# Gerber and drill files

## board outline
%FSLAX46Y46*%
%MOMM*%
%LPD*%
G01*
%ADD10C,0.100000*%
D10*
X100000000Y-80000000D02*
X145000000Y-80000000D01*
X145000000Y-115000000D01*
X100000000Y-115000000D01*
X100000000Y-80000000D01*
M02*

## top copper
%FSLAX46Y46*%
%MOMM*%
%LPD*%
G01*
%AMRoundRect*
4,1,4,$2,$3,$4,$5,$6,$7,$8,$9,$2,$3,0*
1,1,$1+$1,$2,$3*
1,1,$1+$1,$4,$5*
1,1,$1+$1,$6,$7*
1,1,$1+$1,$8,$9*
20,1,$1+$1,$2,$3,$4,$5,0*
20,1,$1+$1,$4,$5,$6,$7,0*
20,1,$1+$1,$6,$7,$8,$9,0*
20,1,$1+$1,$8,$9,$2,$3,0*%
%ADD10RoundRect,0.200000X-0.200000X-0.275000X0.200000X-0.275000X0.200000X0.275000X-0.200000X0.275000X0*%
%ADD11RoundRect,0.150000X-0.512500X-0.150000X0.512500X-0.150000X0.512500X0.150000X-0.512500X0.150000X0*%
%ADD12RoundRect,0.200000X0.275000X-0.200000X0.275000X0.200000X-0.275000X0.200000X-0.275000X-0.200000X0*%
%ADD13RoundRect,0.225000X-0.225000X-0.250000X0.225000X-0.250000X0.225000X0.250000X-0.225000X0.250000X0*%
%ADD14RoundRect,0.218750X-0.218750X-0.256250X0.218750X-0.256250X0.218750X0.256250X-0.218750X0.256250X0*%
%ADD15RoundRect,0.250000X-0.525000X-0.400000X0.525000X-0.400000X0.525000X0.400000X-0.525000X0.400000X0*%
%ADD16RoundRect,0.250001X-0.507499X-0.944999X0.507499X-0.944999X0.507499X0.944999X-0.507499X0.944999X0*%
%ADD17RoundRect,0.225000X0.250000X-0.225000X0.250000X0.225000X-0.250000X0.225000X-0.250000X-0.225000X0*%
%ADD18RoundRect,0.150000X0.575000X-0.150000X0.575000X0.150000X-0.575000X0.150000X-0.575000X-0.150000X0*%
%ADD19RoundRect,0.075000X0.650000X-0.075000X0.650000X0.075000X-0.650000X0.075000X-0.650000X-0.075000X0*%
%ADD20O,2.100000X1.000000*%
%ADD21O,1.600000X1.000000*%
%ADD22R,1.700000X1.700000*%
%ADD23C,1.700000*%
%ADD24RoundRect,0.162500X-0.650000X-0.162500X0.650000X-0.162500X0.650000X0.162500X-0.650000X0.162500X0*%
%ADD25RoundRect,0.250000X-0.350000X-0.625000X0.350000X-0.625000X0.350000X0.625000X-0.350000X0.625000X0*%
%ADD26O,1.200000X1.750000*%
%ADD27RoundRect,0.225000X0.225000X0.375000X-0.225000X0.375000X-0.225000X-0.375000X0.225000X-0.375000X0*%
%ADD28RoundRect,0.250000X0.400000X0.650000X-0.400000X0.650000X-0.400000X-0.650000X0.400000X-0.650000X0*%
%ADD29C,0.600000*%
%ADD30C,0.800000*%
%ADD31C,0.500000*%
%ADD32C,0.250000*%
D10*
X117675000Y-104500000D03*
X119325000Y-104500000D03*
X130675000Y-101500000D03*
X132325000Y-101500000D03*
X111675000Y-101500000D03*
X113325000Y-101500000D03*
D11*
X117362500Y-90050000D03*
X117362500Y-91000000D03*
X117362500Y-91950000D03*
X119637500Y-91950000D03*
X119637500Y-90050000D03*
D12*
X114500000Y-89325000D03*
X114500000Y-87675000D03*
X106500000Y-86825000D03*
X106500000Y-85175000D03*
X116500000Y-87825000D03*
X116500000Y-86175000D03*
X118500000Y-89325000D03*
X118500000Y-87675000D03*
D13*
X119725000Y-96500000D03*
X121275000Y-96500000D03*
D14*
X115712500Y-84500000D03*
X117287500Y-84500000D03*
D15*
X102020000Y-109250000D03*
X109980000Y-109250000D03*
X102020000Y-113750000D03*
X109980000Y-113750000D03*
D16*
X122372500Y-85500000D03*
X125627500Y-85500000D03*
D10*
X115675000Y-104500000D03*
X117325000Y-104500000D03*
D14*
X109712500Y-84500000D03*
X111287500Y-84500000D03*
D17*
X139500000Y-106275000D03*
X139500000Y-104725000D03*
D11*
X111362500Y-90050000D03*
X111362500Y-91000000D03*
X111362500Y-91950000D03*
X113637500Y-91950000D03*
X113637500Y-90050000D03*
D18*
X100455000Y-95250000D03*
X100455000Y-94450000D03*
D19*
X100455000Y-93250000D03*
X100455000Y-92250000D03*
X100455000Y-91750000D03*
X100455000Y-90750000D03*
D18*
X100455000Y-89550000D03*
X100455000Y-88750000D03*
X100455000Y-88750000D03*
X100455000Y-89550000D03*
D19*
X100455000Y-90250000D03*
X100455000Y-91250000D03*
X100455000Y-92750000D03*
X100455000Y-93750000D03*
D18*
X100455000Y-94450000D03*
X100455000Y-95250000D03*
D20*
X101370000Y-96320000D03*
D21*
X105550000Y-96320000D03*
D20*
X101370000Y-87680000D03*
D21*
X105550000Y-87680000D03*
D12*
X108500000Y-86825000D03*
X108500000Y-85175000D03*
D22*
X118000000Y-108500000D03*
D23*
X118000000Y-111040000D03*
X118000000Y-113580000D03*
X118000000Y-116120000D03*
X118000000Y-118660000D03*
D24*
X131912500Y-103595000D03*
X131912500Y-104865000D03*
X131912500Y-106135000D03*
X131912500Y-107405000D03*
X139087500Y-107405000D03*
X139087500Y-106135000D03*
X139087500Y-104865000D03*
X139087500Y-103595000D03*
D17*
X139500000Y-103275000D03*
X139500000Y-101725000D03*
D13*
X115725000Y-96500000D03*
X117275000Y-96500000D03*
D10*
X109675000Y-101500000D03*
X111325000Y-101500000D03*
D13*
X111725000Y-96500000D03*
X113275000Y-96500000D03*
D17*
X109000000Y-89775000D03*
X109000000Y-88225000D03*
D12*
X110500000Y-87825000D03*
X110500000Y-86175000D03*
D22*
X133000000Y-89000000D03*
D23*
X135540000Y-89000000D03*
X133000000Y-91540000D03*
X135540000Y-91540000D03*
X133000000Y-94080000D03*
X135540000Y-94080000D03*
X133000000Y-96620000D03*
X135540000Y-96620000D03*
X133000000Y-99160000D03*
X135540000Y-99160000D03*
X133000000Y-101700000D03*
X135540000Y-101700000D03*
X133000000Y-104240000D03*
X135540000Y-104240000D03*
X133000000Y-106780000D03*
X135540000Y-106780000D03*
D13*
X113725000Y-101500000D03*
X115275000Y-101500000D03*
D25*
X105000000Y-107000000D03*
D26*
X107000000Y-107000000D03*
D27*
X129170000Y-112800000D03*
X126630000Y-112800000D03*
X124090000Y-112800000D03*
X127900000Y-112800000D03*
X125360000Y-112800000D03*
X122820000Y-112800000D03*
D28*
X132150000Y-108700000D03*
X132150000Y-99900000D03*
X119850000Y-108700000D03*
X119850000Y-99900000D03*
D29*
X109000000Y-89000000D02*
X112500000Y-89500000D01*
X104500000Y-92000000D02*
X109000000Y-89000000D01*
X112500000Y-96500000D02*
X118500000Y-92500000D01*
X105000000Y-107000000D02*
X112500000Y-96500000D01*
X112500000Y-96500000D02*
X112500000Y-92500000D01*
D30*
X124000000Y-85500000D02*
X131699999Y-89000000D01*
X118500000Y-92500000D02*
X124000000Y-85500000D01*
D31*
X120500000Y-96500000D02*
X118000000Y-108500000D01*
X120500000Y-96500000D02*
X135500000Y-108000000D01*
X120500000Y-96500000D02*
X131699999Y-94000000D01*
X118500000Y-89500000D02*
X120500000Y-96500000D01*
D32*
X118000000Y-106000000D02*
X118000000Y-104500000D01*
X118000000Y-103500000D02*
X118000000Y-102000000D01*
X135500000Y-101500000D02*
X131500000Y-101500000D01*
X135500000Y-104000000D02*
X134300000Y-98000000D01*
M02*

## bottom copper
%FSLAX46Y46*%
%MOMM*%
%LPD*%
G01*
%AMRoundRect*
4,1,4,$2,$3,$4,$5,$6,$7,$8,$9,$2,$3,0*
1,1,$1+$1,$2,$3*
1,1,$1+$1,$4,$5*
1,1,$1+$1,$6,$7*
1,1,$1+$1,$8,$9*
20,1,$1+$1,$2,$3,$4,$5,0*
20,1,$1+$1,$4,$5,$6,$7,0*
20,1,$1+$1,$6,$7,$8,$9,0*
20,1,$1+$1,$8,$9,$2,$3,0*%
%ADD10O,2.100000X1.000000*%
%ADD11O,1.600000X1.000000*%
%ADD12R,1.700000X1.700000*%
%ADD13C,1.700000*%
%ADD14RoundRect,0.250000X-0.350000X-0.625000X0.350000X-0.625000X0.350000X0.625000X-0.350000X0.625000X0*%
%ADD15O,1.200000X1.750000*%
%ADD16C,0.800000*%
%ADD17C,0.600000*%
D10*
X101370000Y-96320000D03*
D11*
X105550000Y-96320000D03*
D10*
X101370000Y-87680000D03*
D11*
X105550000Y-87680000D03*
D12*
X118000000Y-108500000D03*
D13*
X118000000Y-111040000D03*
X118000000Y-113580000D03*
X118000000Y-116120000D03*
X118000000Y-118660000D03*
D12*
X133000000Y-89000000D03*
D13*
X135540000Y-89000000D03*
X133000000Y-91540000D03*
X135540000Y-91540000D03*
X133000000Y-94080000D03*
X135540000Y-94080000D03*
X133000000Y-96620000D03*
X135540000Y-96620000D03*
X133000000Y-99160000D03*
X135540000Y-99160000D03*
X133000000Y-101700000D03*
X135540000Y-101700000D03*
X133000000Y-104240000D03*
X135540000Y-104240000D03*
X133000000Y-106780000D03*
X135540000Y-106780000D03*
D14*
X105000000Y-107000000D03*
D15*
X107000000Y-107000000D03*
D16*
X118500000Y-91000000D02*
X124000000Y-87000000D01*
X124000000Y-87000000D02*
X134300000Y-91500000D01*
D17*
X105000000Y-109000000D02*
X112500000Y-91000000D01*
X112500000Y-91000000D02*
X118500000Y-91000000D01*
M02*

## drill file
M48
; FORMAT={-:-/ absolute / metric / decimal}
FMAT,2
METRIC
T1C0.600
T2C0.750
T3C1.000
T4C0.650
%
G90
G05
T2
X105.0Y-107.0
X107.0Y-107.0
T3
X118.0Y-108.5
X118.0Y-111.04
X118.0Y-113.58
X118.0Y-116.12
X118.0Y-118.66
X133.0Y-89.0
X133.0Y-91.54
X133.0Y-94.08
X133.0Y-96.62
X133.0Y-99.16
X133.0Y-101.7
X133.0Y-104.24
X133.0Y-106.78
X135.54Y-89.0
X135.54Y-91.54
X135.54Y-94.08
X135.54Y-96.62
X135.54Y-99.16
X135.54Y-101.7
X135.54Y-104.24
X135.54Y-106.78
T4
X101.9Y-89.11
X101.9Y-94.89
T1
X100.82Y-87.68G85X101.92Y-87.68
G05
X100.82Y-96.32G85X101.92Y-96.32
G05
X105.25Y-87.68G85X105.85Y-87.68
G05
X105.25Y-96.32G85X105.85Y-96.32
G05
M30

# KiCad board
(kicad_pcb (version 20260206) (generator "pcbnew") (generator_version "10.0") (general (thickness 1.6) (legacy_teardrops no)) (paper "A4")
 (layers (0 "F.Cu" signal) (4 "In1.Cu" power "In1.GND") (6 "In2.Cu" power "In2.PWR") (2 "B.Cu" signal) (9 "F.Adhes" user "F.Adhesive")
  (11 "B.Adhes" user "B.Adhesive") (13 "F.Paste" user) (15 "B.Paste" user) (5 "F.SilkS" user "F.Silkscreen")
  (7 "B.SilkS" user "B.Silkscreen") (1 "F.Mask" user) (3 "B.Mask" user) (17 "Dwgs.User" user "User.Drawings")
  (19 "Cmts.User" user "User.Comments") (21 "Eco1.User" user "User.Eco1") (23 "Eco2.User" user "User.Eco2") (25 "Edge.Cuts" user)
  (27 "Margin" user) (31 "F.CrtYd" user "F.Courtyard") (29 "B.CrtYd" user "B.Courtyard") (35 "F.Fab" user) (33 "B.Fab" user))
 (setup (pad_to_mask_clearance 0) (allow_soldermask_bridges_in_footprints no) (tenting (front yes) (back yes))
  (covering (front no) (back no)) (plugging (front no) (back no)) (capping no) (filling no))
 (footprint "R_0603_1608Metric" (layer "F.Cu") (at 118.5 104.5)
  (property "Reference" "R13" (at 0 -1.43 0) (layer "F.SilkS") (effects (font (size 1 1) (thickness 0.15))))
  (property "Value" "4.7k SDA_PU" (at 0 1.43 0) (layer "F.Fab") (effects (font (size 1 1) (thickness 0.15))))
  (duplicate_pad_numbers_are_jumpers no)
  (pad "1" smd roundrect (at -0.825 0) (size 0.8 0.95) (layers "F.Cu" "F.Mask" "F.Paste") (roundrect_rratio 0.25))
  (pad "2" smd roundrect (at 0.825 0) (size 0.8 0.95) (layers "F.Cu" "F.Mask" "F.Paste") (roundrect_rratio 0.25)))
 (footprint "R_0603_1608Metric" (layer "F.Cu") (at 131.5 101.5)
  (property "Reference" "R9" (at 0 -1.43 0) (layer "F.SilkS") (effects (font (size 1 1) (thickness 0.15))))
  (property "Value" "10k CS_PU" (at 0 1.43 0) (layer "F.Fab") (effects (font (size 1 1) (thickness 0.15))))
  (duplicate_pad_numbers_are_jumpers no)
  (pad "1" smd roundrect (at -0.825 0) (size 0.8 0.95) (layers "F.Cu" "F.Mask" "F.Paste") (roundrect_rratio 0.25))
  (pad "2" smd roundrect (at 0.825 0) (size 0.8 0.95) (layers "F.Cu" "F.Mask" "F.Paste") (roundrect_rratio 0.25)))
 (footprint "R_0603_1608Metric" (layer "F.Cu") (at 112.5 101.5)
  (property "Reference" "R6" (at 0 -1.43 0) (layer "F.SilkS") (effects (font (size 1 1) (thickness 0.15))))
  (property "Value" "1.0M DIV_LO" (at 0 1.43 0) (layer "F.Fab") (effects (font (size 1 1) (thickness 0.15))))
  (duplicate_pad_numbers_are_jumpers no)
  (pad "1" smd roundrect (at -0.825 0) (size 0.8 0.95) (layers "F.Cu" "F.Mask" "F.Paste") (roundrect_rratio 0.25))
  (pad "2" smd roundrect (at 0.825 0) (size 0.8 0.95) (layers "F.Cu" "F.Mask" "F.Paste") (roundrect_rratio 0.25)))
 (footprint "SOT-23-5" (layer "F.Cu") (at 118.5 91)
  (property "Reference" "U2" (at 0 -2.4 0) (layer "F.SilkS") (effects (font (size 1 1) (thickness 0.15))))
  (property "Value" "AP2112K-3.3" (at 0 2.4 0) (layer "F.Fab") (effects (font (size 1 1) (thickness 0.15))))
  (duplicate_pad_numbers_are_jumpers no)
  (pad "1" smd roundrect (at -1.1375 -0.95) (size 1.325 0.6) (layers "F.Cu" "F.Mask" "F.Paste") (roundrect_rratio 0.25) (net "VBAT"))
  (pad "2" smd roundrect (at -1.1375 0) (size 1.325 0.6) (layers "F.Cu" "F.Mask" "F.Paste") (roundrect_rratio 0.25) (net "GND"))
  (pad "3" smd roundrect (at -1.1375 0.95) (size 1.325 0.6) (layers "F.Cu" "F.Mask" "F.Paste") (roundrect_rratio 0.25) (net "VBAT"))
  (pad "4" smd roundrect (at 1.1375 0.95) (size 1.325 0.6) (layers "F.Cu" "F.Mask" "F.Paste") (roundrect_rratio 0.25))
  (pad "5" smd roundrect (at 1.1375 -0.95) (size 1.325 0.6) (layers "F.Cu" "F.Mask" "F.Paste") (roundrect_rratio 0.25) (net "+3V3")))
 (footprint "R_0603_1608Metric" (layer "F.Cu") (at 114.5 88.5 90)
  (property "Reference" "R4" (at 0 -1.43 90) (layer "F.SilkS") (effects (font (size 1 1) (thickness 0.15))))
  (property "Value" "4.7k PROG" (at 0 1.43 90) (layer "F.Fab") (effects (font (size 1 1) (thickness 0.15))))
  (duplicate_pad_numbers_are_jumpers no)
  (pad "1" smd roundrect (at -0.825 0 90) (size 0.8 0.95) (layers "F.Cu" "F.Mask" "F.Paste") (roundrect_rratio 0.25))
  (pad "2" smd roundrect (at 0.825 0 90) (size 0.8 0.95) (layers "F.Cu" "F.Mask" "F.Paste") (roundrect_rratio 0.25)))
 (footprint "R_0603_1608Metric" (layer "F.Cu") (at 106.5 86 90)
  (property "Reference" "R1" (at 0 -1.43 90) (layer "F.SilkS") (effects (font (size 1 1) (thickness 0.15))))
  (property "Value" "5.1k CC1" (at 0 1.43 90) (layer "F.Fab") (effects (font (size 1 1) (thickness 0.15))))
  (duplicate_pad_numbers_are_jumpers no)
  (pad "1" smd roundrect (at -0.825 0 90) (size 0.8 0.95) (layers "F.Cu" "F.Mask" "F.Paste") (roundrect_rratio 0.25))
  (pad "2" smd roundrect (at 0.825 0 90) (size 0.8 0.95) (layers "F.Cu" "F.Mask" "F.Paste") (roundrect_rratio 0.25)))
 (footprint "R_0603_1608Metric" (layer "F.Cu") (at 116.5 87 90)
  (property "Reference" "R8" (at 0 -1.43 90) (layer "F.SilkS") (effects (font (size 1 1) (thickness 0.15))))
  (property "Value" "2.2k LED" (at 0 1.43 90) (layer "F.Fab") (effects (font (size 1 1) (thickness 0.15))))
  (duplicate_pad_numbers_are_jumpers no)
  (pad "1" smd roundrect (at -0.825 0 90) (size 0.8 0.95) (layers "F.Cu" "F.Mask" "F.Paste") (roundrect_rratio 0.25))
  (pad "2" smd roundrect (at 0.825 0 90) (size 0.8 0.95) (layers "F.Cu" "F.Mask" "F.Paste") (roundrect_rratio 0.25)))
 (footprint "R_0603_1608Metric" (layer "F.Cu") (at 118.5 88.5 90)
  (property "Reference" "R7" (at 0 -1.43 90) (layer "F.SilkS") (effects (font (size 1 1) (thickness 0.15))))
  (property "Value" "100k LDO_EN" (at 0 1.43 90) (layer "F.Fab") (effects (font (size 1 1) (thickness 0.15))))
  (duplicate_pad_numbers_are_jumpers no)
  (pad "1" smd roundrect (at -0.825 0 90) (size 0.8 0.95) (layers "F.Cu" "F.Mask" "F.Paste") (roundrect_rratio 0.25))
  (pad "2" smd roundrect (at 0.825 0 90) (size 0.8 0.95) (layers "F.Cu" "F.Mask" "F.Paste") (roundrect_rratio 0.25)))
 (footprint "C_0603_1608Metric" (layer "F.Cu") (at 120.5 96.5)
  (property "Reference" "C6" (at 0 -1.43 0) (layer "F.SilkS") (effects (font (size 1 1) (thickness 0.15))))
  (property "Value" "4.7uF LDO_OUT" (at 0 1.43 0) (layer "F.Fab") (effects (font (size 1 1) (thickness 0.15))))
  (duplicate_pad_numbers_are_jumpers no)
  (pad "1" smd roundrect (at -0.775 0) (size 0.9 0.95) (layers "F.Cu" "F.Mask" "F.Paste") (roundrect_rratio 0.25) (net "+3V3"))
  (pad "2" smd roundrect (at 0.775 0) (size 0.9 0.95) (layers "F.Cu" "F.Mask" "F.Paste") (roundrect_rratio 0.25) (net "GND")))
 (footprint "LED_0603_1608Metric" (layer "F.Cu") (at 116.5 84.5)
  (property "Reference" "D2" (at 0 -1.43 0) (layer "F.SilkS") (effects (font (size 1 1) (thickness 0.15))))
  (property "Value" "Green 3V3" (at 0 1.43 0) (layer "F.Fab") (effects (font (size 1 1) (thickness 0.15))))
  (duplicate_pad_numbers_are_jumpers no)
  (pad "1" smd roundrect (at -0.7875 0) (size 0.875 0.95) (layers "F.Cu" "F.Mask" "F.Paste") (roundrect_rratio 0.25))
  (pad "2" smd roundrect (at 0.7875 0) (size 0.875 0.95) (layers "F.Cu" "F.Mask" "F.Paste") (roundrect_rratio 0.25)))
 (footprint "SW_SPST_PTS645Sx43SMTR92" (layer "F.Cu") (at 106 111.5)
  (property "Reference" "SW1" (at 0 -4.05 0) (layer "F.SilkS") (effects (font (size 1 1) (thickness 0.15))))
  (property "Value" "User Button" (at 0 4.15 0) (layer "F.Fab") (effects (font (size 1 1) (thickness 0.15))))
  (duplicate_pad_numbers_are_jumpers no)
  (pad "1" smd roundrect (at -3.98 -2.25) (size 1.55 1.3) (layers "F.Cu" "F.Mask" "F.Paste") (roundrect_rratio 0.1923076923))
  (pad "1" smd roundrect (at 3.98 -2.25) (size 1.55 1.3) (layers "F.Cu" "F.Mask" "F.Paste") (roundrect_rratio 0.1923076923))
  (pad "2" smd roundrect (at -3.98 2.25) (size 1.55 1.3) (layers "F.Cu" "F.Mask" "F.Paste") (roundrect_rratio 0.1923076923))
  (pad "2" smd roundrect (at 3.98 2.25) (size 1.55 1.3) (layers "F.Cu" "F.Mask" "F.Paste") (roundrect_rratio 0.1923076923)))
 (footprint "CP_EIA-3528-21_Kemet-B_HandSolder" (layer "F.Cu") (at 124 85.5)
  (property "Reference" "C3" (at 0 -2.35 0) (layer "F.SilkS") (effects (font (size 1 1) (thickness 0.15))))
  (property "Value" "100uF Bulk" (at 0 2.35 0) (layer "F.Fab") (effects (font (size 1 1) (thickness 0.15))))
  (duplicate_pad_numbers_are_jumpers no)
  (pad "1" smd roundrect (at -1.6275 0) (size 1.515 2.39) (layers "F.Cu" "F.Mask" "F.Paste") (roundrect_rratio 0.165017) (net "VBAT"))
  (pad "2" smd roundrect (at 1.6275 0) (size 1.515 2.39) (layers "F.Cu" "F.Mask" "F.Paste") (roundrect_rratio 0.165017) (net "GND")))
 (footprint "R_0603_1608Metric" (layer "F.Cu") (at 116.5 104.5)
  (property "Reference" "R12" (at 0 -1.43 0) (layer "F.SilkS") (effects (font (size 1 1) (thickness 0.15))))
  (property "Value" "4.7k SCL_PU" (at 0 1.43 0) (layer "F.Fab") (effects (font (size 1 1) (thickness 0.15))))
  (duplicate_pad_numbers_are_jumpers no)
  (pad "1" smd roundrect (at -0.825 0) (size 0.8 0.95) (layers "F.Cu" "F.Mask" "F.Paste") (roundrect_rratio 0.25))
  (pad "2" smd roundrect (at 0.825 0) (size 0.8 0.95) (layers "F.Cu" "F.Mask" "F.Paste") (roundrect_rratio 0.25)))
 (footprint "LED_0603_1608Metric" (layer "F.Cu") (at 110.5 84.5)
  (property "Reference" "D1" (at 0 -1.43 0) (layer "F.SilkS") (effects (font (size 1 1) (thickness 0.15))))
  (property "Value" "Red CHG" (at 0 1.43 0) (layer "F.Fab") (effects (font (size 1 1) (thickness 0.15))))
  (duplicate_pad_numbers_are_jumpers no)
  (pad "1" smd roundrect (at -0.7875 0) (size 0.875 0.95) (layers "F.Cu" "F.Mask" "F.Paste") (roundrect_rratio 0.25))
  (pad "2" smd roundrect (at 0.7875 0) (size 0.875 0.95) (layers "F.Cu" "F.Mask" "F.Paste") (roundrect_rratio 0.25)))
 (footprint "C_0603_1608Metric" (layer "F.Cu") (at 139.5 105.5 90)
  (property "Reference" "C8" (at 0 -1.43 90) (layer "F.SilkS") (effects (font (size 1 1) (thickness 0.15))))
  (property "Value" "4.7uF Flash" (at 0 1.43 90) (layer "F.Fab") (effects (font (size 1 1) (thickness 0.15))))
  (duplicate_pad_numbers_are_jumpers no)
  (pad "1" smd roundrect (at -0.775 0 90) (size 0.9 0.95) (layers "F.Cu" "F.Mask" "F.Paste") (roundrect_rratio 0.25) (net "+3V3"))
  (pad "2" smd roundrect (at 0.775 0 90) (size 0.9 0.95) (layers "F.Cu" "F.Mask" "F.Paste") (roundrect_rratio 0.25) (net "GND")))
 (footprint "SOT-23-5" (layer "F.Cu") (at 112.5 91)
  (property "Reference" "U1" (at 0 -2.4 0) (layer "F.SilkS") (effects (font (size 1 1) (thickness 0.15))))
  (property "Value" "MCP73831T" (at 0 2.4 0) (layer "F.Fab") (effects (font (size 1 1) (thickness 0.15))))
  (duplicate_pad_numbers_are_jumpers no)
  (pad "1" smd roundrect (at -1.1375 -0.95) (size 1.325 0.6) (layers "F.Cu" "F.Mask" "F.Paste") (roundrect_rratio 0.25) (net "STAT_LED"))
  (pad "2" smd roundrect (at -1.1375 0) (size 1.325 0.6) (layers "F.Cu" "F.Mask" "F.Paste") (roundrect_rratio 0.25) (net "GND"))
  (pad "3" smd roundrect (at -1.1375 0.95) (size 1.325 0.6) (layers "F.Cu" "F.Mask" "F.Paste") (roundrect_rratio 0.25) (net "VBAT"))
  (pad "4" smd roundrect (at 1.1375 0.95) (size 1.325 0.6) (layers "F.Cu" "F.Mask" "F.Paste") (roundrect_rratio 0.25) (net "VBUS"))
  (pad "5" smd roundrect (at 1.1375 -0.95) (size 1.325 0.6) (layers "F.Cu" "F.Mask" "F.Paste") (roundrect_rratio 0.25) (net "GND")))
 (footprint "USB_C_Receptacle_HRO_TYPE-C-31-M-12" (layer "F.Cu") (at 104.5 92 90)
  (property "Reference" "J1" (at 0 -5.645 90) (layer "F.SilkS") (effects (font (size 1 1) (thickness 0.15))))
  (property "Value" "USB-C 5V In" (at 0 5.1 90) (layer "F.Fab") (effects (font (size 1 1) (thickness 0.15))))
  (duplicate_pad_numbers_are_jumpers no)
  (pad "" np_thru_hole circle (at -2.89 -2.6 90) (size 0.65 0.65) (drill 0.65) (layers "*.Cu" "*.Mask"))
  (pad "" np_thru_hole circle (at 2.89 -2.6 90) (size 0.65 0.65) (drill 0.65) (layers "*.Cu" "*.Mask"))
  (pad "A1" smd roundrect (at -3.25 -4.045 90) (size 0.6 1.45) (layers "F.Cu" "F.Mask" "F.Paste") (roundrect_rratio 0.25))
  (pad "A4" smd roundrect (at -2.45 -4.045 90) (size 0.6 1.45) (layers "F.Cu" "F.Mask" "F.Paste") (roundrect_rratio 0.25))
  (pad "A5" smd roundrect (at -1.25 -4.045 90) (size 0.3 1.45) (layers "F.Cu" "F.Mask" "F.Paste") (roundrect_rratio 0.25))
  (pad "A6" smd roundrect (at -0.25 -4.045 90) (size 0.3 1.45) (layers "F.Cu" "F.Mask" "F.Paste") (roundrect_rratio 0.25))
  (pad "A7" smd roundrect (at 0.25 -4.045 90) (size 0.3 1.45) (layers "F.Cu" "F.Mask" "F.Paste") (roundrect_rratio 0.25))
  (pad "A8" smd roundrect (at 1.25 -4.045 90) (size 0.3 1.45) (layers "F.Cu" "F.Mask" "F.Paste") (roundrect_rratio 0.25))
  (pad "A9" smd roundrect (at 2.45 -4.045 90) (size 0.6 1.45) (layers "F.Cu" "F.Mask" "F.Paste") (roundrect_rratio 0.25))
  (pad "A12" smd roundrect (at 3.25 -4.045 90) (size 0.6 1.45) (layers "F.Cu" "F.Mask" "F.Paste") (roundrect_rratio 0.25))
  (pad "B1" smd roundrect (at 3.25 -4.045 90) (size 0.6 1.45) (layers "F.Cu" "F.Mask" "F.Paste") (roundrect_rratio 0.25))
  (pad "B4" smd roundrect (at 2.45 -4.045 90) (size 0.6 1.45) (layers "F.Cu" "F.Mask" "F.Paste") (roundrect_rratio 0.25))
  (pad "B5" smd roundrect (at 1.75 -4.045 90) (size 0.3 1.45) (layers "F.Cu" "F.Mask" "F.Paste") (roundrect_rratio 0.25))
  (pad "B6" smd roundrect (at 0.75 -4.045 90) (size 0.3 1.45) (layers "F.Cu" "F.Mask" "F.Paste") (roundrect_rratio 0.25))
  (pad "B7" smd roundrect (at -0.75 -4.045 90) (size 0.3 1.45) (layers "F.Cu" "F.Mask" "F.Paste") (roundrect_rratio 0.25))
  (pad "B8" smd roundrect (at -1.75 -4.045 90) (size 0.3 1.45) (layers "F.Cu" "F.Mask" "F.Paste") (roundrect_rratio 0.25))
  (pad "B9" smd roundrect (at -2.45 -4.045 90) (size 0.6 1.45) (layers "F.Cu" "F.Mask" "F.Paste") (roundrect_rratio 0.25))
  (pad "B12" smd roundrect (at -3.25 -4.045 90) (size 0.6 1.45) (layers "F.Cu" "F.Mask" "F.Paste") (roundrect_rratio 0.25))
  (pad "SH" thru_hole oval (at -4.32 -3.13 90) (size 1 2.1) (drill oval 0.6 1.7) (layers "*.Cu" "*.Mask") (remove_unused_layers no))
  (pad "SH" thru_hole oval (at -4.32 1.05 90) (size 1 1.6) (drill oval 0.6 1.2) (layers "*.Cu" "*.Mask") (remove_unused_layers no))
  (pad "SH" thru_hole oval (at 4.32 -3.13 90) (size 1 2.1) (drill oval 0.6 1.7) (layers "*.Cu" "*.Mask") (remove_unused_layers no))
  (pad "SH" thru_hole oval (at 4.32 1.05 90) (size 1 1.6) (drill oval 0.6 1.2) (layers "*.Cu" "*.Mask") (remove_unused_layers no)))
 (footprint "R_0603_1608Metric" (layer "F.Cu") (at 108.5 86 90)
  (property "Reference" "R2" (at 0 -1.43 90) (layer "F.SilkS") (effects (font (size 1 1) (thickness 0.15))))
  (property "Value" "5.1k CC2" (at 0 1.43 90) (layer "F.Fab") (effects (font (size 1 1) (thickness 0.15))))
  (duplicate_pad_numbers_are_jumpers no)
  (pad "1" smd roundrect (at -0.825 0 90) (size 0.8 0.95) (layers "F.Cu" "F.Mask" "F.Paste") (roundrect_rratio 0.25))
  (pad "2" smd roundrect (at 0.825 0 90) (size 0.8 0.95) (layers "F.Cu" "F.Mask" "F.Paste") (roundrect_rratio 0.25)))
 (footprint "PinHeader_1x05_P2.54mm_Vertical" (layer "F.Cu") (at 118 108.5)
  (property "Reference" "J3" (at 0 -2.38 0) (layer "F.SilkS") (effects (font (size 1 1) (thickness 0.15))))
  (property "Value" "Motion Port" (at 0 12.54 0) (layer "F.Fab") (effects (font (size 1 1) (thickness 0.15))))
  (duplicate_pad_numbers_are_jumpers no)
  (pad "1" thru_hole rect (at 0 0) (size 1.7 1.7) (drill 1) (layers "*.Cu" "*.Mask") (remove_unused_layers no) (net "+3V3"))
  (pad "2" thru_hole circle (at 0 2.54) (size 1.7 1.7) (drill 1) (layers "*.Cu" "*.Mask") (remove_unused_layers no) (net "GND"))
  (pad "3" thru_hole circle (at 0 5.08) (size 1.7 1.7) (drill 1) (layers "*.Cu" "*.Mask") (remove_unused_layers no) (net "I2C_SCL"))
  (pad "4" thru_hole circle (at 0 7.62) (size 1.7 1.7) (drill 1) (layers "*.Cu" "*.Mask") (remove_unused_layers no) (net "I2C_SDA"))
  (pad "5" thru_hole circle (at 0 10.16) (size 1.7 1.7) (drill 1) (layers "*.Cu" "*.Mask") (remove_unused_layers no) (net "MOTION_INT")))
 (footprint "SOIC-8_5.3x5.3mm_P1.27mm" (layer "F.Cu") (at 135.5 105.5)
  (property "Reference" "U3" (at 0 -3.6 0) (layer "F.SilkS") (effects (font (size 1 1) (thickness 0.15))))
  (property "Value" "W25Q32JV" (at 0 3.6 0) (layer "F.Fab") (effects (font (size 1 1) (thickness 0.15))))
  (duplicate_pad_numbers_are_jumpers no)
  (pad "1" smd roundrect (at -3.5875 -1.905) (size 1.625 0.65) (layers "F.Cu" "F.Mask" "F.Paste") (roundrect_rratio 0.25) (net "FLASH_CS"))
  (pad "2" smd roundrect (at -3.5875 -0.635) (size 1.625 0.65) (layers "F.Cu" "F.Mask" "F.Paste") (roundrect_rratio 0.25) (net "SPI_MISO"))
  (pad "3" smd roundrect (at -3.5875 0.635) (size 1.625 0.65) (layers "F.Cu" "F.Mask" "F.Paste") (roundrect_rratio 0.25) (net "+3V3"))
  (pad "4" smd roundrect (at -3.5875 1.905) (size 1.625 0.65) (layers "F.Cu" "F.Mask" "F.Paste") (roundrect_rratio 0.25) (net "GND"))
  (pad "5" smd roundrect (at 3.5875 1.905) (size 1.625 0.65) (layers "F.Cu" "F.Mask" "F.Paste") (roundrect_rratio 0.25) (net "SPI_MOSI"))
  (pad "6" smd roundrect (at 3.5875 0.635) (size 1.625 0.65) (layers "F.Cu" "F.Mask" "F.Paste") (roundrect_rratio 0.25) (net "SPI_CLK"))
  (pad "7" smd roundrect (at 3.5875 -0.635) (size 1.625 0.65) (layers "F.Cu" "F.Mask" "F.Paste") (roundrect_rratio 0.25) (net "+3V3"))
  (pad "8" smd roundrect (at 3.5875 -1.905) (size 1.625 0.65) (layers "F.Cu" "F.Mask" "F.Paste") (roundrect_rratio 0.25) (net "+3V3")))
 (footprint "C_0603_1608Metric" (layer "F.Cu") (at 139.5 102.5 90)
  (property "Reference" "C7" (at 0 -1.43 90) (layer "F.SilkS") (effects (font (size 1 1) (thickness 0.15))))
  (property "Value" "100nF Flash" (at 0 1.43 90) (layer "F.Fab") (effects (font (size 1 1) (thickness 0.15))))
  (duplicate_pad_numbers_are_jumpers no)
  (pad "1" smd roundrect (at -0.775 0 90) (size 0.9 0.95) (layers "F.Cu" "F.Mask" "F.Paste") (roundrect_rratio 0.25) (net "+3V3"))
  (pad "2" smd roundrect (at 0.775 0 90) (size 0.9 0.95) (layers "F.Cu" "F.Mask" "F.Paste") (roundrect_rratio 0.25) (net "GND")))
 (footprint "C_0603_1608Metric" (layer "F.Cu") (at 116.5 96.5)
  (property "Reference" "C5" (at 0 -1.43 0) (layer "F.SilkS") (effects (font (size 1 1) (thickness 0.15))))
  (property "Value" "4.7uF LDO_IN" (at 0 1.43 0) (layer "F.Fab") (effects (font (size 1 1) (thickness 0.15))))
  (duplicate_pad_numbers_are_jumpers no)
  (pad "1" smd roundrect (at -0.775 0) (size 0.9 0.95) (layers "F.Cu" "F.Mask" "F.Paste") (roundrect_rratio 0.25) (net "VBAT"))
  (pad "2" smd roundrect (at 0.775 0) (size 0.9 0.95) (layers "F.Cu" "F.Mask" "F.Paste") (roundrect_rratio 0.25) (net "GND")))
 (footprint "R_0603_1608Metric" (layer "F.Cu") (at 110.5 101.5)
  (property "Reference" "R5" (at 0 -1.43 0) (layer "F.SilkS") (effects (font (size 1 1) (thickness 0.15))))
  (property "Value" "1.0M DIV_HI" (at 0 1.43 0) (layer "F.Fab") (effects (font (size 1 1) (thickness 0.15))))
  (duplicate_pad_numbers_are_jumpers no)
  (pad "1" smd roundrect (at -0.825 0) (size 0.8 0.95) (layers "F.Cu" "F.Mask" "F.Paste") (roundrect_rratio 0.25))
  (pad "2" smd roundrect (at 0.825 0) (size 0.8 0.95) (layers "F.Cu" "F.Mask" "F.Paste") (roundrect_rratio 0.25)))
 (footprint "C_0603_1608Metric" (layer "F.Cu") (at 112.5 96.5)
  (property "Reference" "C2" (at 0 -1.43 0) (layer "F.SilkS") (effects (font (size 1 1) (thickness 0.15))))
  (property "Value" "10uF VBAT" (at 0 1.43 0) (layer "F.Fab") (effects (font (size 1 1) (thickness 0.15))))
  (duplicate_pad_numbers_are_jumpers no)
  (pad "1" smd roundrect (at -0.775 0) (size 0.9 0.95) (layers "F.Cu" "F.Mask" "F.Paste") (roundrect_rratio 0.25) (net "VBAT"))
  (pad "2" smd roundrect (at 0.775 0) (size 0.9 0.95) (layers "F.Cu" "F.Mask" "F.Paste") (roundrect_rratio 0.25) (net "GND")))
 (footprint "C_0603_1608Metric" (layer "F.Cu") (at 109 89 90)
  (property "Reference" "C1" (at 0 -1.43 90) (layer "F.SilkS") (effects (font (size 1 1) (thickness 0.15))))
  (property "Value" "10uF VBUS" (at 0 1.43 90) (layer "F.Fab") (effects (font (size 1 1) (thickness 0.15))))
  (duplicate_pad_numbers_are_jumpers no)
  (pad "1" smd roundrect (at -0.775 0 90) (size 0.9 0.95) (layers "F.Cu" "F.Mask" "F.Paste") (roundrect_rratio 0.25) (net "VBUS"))
  (pad "2" smd roundrect (at 0.775 0 90) (size 0.9 0.95) (layers "F.Cu" "F.Mask" "F.Paste") (roundrect_rratio 0.25) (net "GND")))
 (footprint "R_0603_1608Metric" (layer "F.Cu") (at 110.5 87 90)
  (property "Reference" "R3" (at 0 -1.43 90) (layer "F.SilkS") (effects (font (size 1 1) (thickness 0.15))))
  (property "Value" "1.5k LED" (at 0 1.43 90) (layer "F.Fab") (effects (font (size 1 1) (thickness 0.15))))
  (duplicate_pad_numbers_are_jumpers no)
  (pad "1" smd roundrect (at -0.825 0 90) (size 0.8 0.95) (layers "F.Cu" "F.Mask" "F.Paste") (roundrect_rratio 0.25))
  (pad "2" smd roundrect (at 0.825 0 90) (size 0.8 0.95) (layers "F.Cu" "F.Mask" "F.Paste") (roundrect_rratio 0.25)))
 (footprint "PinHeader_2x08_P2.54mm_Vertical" (layer "F.Cu") (at 133 89)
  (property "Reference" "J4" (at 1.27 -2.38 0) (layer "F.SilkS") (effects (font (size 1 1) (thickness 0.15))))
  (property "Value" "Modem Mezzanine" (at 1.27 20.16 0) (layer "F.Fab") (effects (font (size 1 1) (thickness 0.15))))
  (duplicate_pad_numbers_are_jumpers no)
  (pad "1" thru_hole rect (at 0 0) (size 1.7 1.7) (drill 1) (layers "*.Cu" "*.Mask") (remove_unused_layers no) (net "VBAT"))
  (pad "2" thru_hole circle (at 2.54 0) (size 1.7 1.7) (drill 1) (layers "*.Cu" "*.Mask") (remove_unused_layers no) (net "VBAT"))
  (pad "3" thru_hole circle (at 0 2.54) (size 1.7 1.7) (drill 1) (layers "*.Cu" "*.Mask") (remove_unused_layers no) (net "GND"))
  (pad "4" thru_hole circle (at 2.54 2.54) (size 1.7 1.7) (drill 1) (layers "*.Cu" "*.Mask") (remove_unused_layers no) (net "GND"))
  (pad "5" thru_hole circle (at 0 5.08) (size 1.7 1.7) (drill 1) (layers "*.Cu" "*.Mask") (remove_unused_layers no) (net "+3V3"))
  (pad "6" thru_hole circle (at 2.54 5.08) (size 1.7 1.7) (drill 1) (layers "*.Cu" "*.Mask") (remove_unused_layers no) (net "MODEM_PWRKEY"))
  (pad "7" thru_hole circle (at 0 7.62) (size 1.7 1.7) (drill 1) (layers "*.Cu" "*.Mask") (remove_unused_layers no) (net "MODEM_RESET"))
  (pad "8" thru_hole circle (at 2.54 7.62) (size 1.7 1.7) (drill 1) (layers "*.Cu" "*.Mask") (remove_unused_layers no) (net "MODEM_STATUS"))
  (pad "9" thru_hole circle (at 0 10.16) (size 1.7 1.7) (drill 1) (layers "*.Cu" "*.Mask") (remove_unused_layers no) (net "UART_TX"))
  (pad "10" thru_hole circle (at 2.54 10.16) (size 1.7 1.7) (drill 1) (layers "*.Cu" "*.Mask") (remove_unused_layers no) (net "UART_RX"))
  (pad "11" thru_hole circle (at 0 12.7) (size 1.7 1.7) (drill 1) (layers "*.Cu" "*.Mask") (remove_unused_layers no) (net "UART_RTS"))
  (pad "12" thru_hole circle (at 2.54 12.7) (size 1.7 1.7) (drill 1) (layers "*.Cu" "*.Mask") (remove_unused_layers no) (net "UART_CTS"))
  (pad "13" thru_hole circle (at 0 15.24) (size 1.7 1.7) (drill 1) (layers "*.Cu" "*.Mask") (remove_unused_layers no) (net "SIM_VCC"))
  (pad "14" thru_hole circle (at 2.54 15.24) (size 1.7 1.7) (drill 1) (layers "*.Cu" "*.Mask") (remove_unused_layers no) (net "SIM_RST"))
  (pad "15" thru_hole circle (at 0 17.78) (size 1.7 1.7) (drill 1) (layers "*.Cu" "*.Mask") (remove_unused_layers no) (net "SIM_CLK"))
  (pad "16" thru_hole circle (at 2.54 17.78) (size 1.7 1.7) (drill 1) (layers "*.Cu" "*.Mask") (remove_unused_layers no) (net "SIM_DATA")))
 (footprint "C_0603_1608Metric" (layer "F.Cu") (at 114.5 101.5)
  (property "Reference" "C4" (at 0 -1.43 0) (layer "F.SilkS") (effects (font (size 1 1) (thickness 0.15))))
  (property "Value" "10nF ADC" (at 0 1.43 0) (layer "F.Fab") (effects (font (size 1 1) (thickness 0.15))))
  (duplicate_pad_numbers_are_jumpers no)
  (pad "1" smd roundrect (at -0.775 0) (size 0.9 0.95) (layers "F.Cu" "F.Mask" "F.Paste") (roundrect_rratio 0.25))
  (pad "2" smd roundrect (at 0.775 0) (size 0.9 0.95) (layers "F.Cu" "F.Mask" "F.Paste") (roundrect_rratio 0.25)))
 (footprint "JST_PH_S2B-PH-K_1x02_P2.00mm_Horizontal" (layer "F.Cu") (at 105 107)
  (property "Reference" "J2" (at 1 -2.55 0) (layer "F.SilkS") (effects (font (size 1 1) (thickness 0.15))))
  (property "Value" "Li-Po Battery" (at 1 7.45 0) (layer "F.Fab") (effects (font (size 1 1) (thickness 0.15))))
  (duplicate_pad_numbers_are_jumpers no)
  (pad "1" thru_hole roundrect (at 0 0) (size 1.2 1.75) (drill 0.75) (layers "*.Cu" "*.Mask") (remove_unused_layers no)
   (roundrect_rratio 0.208333) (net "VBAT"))
  (pad "2" thru_hole oval (at 2 0) (size 1.2 1.75) (drill 0.75) (layers "*.Cu" "*.Mask") (remove_unused_layers no) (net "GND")))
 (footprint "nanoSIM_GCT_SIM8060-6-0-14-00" (layer "F.Cu") (at 126 106 180)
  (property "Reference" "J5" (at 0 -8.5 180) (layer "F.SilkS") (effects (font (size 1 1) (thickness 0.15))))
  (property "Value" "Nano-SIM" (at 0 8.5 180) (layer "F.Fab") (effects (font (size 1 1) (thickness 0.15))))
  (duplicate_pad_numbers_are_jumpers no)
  (pad "1" smd roundrect (at -3.17 -6.8 180) (size 0.9 1.2) (layers "F.Cu" "F.Mask" "F.Paste") (roundrect_rratio 0.25)
   (thermal_bridge_angle 45))
  (pad "2" smd roundrect (at -0.63 -6.8 180) (size 0.9 1.2) (layers "F.Cu" "F.Mask" "F.Paste") (roundrect_rratio 0.25)
   (thermal_bridge_angle 45))
  (pad "3" smd roundrect (at 1.91 -6.8 180) (size 0.9 1.2) (layers "F.Cu" "F.Mask" "F.Paste") (roundrect_rratio 0.25)
   (thermal_bridge_angle 45))
  (pad "5" smd roundrect (at -1.9 -6.8 180) (size 0.9 1.2) (layers "F.Cu" "F.Mask" "F.Paste") (roundrect_rratio 0.25)
   (thermal_bridge_angle 45))
  (pad "6" smd roundrect (at 0.64 -6.8 180) (size 0.9 1.2) (layers "F.Cu" "F.Mask" "F.Paste") (roundrect_rratio 0.25)
   (thermal_bridge_angle 45))
  (pad "7" smd roundrect (at 3.18 -6.8 180) (size 0.9 1.2) (layers "F.Cu" "F.Mask" "F.Paste") (roundrect_rratio 0.25)
   (thermal_bridge_angle 45))
  (pad "SH" smd roundrect (at -6.15 -2.7 180) (size 1.3 1.8) (layers "F.Cu" "F.Mask" "F.Paste") (roundrect_rratio 0.1923076923)
   (thermal_bridge_angle 45))
  (pad "SH" smd roundrect (at -6.15 6.1 180) (size 1.3 1.8) (layers "F.Cu" "F.Mask" "F.Paste") (roundrect_rratio 0.1923076923)
   (thermal_bridge_angle 45))
  (pad "SH" smd roundrect (at 6.15 -2.7 180) (size 1.3 1.8) (layers "F.Cu" "F.Mask" "F.Paste") (roundrect_rratio 0.1923076923)
   (thermal_bridge_angle 45))
  (pad "SH" smd roundrect (at 6.15 6.1 180) (size 1.3 1.8) (layers "F.Cu" "F.Mask" "F.Paste") (roundrect_rratio 0.1923076923)
   (thermal_bridge_angle 45))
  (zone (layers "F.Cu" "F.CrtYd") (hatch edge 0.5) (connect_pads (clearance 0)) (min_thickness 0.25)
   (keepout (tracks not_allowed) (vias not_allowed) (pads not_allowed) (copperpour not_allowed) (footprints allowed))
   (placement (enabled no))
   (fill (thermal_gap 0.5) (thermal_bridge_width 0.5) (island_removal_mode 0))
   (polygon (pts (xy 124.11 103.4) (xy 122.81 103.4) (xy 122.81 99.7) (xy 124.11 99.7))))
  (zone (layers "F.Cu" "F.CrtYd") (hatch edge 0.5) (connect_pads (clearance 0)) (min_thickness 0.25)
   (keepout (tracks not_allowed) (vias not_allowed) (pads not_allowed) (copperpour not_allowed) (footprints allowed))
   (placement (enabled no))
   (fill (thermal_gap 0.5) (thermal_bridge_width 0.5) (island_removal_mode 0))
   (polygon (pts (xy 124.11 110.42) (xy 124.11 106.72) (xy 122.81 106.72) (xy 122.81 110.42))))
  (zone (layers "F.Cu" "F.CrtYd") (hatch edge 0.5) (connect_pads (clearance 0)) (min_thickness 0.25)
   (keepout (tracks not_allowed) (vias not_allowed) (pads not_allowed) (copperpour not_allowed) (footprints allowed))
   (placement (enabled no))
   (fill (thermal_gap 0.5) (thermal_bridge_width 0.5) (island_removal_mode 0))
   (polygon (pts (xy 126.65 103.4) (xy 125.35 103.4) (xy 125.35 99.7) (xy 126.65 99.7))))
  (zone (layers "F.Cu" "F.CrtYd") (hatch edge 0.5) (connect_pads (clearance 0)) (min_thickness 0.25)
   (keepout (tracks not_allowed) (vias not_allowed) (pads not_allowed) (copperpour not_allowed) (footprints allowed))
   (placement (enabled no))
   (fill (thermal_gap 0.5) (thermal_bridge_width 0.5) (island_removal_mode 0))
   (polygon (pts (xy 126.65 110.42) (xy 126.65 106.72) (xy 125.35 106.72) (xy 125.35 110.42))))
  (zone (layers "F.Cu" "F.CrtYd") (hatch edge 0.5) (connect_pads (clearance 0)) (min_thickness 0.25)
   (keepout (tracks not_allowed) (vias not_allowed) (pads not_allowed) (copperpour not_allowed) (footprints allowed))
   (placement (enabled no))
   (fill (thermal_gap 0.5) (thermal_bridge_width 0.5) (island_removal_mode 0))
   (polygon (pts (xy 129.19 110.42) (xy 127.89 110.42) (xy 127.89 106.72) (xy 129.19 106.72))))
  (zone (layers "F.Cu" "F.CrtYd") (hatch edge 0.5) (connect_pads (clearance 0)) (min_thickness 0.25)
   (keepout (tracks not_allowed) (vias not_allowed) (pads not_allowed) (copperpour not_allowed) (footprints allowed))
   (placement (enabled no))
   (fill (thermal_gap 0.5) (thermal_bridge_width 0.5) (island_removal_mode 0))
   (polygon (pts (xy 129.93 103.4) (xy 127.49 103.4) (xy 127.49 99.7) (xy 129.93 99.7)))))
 (gr_rect (start 100 80) (end 145 115) (stroke (width 0.1) (type solid)) (fill no) (layer "Edge.Cuts"))
 (segment (start 118.5 91) (end 124 87) (width 0.8) (layer "B.Cu") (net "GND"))
 (segment (start 124 87) (end 134.3 91.5) (width 0.8) (layer "B.Cu") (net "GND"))
 (segment (start 105 109) (end 112.5 91) (width 0.6) (layer "B.Cu") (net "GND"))
 (segment (start 112.5 91) (end 118.5 91) (width 0.6) (layer "B.Cu") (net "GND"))
 (segment (start 109 89) (end 112.5 89.5) (width 0.6) (layer "F.Cu") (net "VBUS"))
 (segment (start 104.5 92) (end 109 89) (width 0.6) (layer "F.Cu") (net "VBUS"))
 (segment (start 112.5 96.5) (end 118.5 92.5) (width 0.6) (layer "F.Cu") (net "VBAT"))
 (segment (start 105 107) (end 112.5 96.5) (width 0.6) (layer "F.Cu") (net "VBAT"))
 (segment (start 112.5 96.5) (end 112.5 92.5) (width 0.6) (layer "F.Cu") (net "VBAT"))
 (segment (start 124 85.5) (end 131.699999 89) (width 0.8) (layer "F.Cu") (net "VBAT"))
 (segment (start 118.5 92.5) (end 124 85.5) (width 0.8) (layer "F.Cu") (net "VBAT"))
 (segment (start 120.5 96.5) (end 118 108.5) (width 0.5) (layer "F.Cu") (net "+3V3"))
 (segment (start 120.5 96.5) (end 135.5 108) (width 0.5) (layer "F.Cu") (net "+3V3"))
 (segment (start 120.5 96.5) (end 131.699999 94) (width 0.5) (layer "F.Cu") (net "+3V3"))
 (segment (start 118.5 89.5) (end 120.5 96.5) (width 0.5) (layer "F.Cu") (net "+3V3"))
 (segment (start 118 106) (end 118 104.5) (width 0.25) (layer "F.Cu") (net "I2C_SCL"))
 (segment (start 118 103.5) (end 118 102) (width 0.25) (layer "F.Cu") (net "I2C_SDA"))
 (segment (start 135.5 101.5) (end 131.5 101.5) (width 0.25) (layer "F.Cu") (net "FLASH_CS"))
 (segment (start 135.5 104) (end 134.3 98) (width 0.25) (layer "F.Cu") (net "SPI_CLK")))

